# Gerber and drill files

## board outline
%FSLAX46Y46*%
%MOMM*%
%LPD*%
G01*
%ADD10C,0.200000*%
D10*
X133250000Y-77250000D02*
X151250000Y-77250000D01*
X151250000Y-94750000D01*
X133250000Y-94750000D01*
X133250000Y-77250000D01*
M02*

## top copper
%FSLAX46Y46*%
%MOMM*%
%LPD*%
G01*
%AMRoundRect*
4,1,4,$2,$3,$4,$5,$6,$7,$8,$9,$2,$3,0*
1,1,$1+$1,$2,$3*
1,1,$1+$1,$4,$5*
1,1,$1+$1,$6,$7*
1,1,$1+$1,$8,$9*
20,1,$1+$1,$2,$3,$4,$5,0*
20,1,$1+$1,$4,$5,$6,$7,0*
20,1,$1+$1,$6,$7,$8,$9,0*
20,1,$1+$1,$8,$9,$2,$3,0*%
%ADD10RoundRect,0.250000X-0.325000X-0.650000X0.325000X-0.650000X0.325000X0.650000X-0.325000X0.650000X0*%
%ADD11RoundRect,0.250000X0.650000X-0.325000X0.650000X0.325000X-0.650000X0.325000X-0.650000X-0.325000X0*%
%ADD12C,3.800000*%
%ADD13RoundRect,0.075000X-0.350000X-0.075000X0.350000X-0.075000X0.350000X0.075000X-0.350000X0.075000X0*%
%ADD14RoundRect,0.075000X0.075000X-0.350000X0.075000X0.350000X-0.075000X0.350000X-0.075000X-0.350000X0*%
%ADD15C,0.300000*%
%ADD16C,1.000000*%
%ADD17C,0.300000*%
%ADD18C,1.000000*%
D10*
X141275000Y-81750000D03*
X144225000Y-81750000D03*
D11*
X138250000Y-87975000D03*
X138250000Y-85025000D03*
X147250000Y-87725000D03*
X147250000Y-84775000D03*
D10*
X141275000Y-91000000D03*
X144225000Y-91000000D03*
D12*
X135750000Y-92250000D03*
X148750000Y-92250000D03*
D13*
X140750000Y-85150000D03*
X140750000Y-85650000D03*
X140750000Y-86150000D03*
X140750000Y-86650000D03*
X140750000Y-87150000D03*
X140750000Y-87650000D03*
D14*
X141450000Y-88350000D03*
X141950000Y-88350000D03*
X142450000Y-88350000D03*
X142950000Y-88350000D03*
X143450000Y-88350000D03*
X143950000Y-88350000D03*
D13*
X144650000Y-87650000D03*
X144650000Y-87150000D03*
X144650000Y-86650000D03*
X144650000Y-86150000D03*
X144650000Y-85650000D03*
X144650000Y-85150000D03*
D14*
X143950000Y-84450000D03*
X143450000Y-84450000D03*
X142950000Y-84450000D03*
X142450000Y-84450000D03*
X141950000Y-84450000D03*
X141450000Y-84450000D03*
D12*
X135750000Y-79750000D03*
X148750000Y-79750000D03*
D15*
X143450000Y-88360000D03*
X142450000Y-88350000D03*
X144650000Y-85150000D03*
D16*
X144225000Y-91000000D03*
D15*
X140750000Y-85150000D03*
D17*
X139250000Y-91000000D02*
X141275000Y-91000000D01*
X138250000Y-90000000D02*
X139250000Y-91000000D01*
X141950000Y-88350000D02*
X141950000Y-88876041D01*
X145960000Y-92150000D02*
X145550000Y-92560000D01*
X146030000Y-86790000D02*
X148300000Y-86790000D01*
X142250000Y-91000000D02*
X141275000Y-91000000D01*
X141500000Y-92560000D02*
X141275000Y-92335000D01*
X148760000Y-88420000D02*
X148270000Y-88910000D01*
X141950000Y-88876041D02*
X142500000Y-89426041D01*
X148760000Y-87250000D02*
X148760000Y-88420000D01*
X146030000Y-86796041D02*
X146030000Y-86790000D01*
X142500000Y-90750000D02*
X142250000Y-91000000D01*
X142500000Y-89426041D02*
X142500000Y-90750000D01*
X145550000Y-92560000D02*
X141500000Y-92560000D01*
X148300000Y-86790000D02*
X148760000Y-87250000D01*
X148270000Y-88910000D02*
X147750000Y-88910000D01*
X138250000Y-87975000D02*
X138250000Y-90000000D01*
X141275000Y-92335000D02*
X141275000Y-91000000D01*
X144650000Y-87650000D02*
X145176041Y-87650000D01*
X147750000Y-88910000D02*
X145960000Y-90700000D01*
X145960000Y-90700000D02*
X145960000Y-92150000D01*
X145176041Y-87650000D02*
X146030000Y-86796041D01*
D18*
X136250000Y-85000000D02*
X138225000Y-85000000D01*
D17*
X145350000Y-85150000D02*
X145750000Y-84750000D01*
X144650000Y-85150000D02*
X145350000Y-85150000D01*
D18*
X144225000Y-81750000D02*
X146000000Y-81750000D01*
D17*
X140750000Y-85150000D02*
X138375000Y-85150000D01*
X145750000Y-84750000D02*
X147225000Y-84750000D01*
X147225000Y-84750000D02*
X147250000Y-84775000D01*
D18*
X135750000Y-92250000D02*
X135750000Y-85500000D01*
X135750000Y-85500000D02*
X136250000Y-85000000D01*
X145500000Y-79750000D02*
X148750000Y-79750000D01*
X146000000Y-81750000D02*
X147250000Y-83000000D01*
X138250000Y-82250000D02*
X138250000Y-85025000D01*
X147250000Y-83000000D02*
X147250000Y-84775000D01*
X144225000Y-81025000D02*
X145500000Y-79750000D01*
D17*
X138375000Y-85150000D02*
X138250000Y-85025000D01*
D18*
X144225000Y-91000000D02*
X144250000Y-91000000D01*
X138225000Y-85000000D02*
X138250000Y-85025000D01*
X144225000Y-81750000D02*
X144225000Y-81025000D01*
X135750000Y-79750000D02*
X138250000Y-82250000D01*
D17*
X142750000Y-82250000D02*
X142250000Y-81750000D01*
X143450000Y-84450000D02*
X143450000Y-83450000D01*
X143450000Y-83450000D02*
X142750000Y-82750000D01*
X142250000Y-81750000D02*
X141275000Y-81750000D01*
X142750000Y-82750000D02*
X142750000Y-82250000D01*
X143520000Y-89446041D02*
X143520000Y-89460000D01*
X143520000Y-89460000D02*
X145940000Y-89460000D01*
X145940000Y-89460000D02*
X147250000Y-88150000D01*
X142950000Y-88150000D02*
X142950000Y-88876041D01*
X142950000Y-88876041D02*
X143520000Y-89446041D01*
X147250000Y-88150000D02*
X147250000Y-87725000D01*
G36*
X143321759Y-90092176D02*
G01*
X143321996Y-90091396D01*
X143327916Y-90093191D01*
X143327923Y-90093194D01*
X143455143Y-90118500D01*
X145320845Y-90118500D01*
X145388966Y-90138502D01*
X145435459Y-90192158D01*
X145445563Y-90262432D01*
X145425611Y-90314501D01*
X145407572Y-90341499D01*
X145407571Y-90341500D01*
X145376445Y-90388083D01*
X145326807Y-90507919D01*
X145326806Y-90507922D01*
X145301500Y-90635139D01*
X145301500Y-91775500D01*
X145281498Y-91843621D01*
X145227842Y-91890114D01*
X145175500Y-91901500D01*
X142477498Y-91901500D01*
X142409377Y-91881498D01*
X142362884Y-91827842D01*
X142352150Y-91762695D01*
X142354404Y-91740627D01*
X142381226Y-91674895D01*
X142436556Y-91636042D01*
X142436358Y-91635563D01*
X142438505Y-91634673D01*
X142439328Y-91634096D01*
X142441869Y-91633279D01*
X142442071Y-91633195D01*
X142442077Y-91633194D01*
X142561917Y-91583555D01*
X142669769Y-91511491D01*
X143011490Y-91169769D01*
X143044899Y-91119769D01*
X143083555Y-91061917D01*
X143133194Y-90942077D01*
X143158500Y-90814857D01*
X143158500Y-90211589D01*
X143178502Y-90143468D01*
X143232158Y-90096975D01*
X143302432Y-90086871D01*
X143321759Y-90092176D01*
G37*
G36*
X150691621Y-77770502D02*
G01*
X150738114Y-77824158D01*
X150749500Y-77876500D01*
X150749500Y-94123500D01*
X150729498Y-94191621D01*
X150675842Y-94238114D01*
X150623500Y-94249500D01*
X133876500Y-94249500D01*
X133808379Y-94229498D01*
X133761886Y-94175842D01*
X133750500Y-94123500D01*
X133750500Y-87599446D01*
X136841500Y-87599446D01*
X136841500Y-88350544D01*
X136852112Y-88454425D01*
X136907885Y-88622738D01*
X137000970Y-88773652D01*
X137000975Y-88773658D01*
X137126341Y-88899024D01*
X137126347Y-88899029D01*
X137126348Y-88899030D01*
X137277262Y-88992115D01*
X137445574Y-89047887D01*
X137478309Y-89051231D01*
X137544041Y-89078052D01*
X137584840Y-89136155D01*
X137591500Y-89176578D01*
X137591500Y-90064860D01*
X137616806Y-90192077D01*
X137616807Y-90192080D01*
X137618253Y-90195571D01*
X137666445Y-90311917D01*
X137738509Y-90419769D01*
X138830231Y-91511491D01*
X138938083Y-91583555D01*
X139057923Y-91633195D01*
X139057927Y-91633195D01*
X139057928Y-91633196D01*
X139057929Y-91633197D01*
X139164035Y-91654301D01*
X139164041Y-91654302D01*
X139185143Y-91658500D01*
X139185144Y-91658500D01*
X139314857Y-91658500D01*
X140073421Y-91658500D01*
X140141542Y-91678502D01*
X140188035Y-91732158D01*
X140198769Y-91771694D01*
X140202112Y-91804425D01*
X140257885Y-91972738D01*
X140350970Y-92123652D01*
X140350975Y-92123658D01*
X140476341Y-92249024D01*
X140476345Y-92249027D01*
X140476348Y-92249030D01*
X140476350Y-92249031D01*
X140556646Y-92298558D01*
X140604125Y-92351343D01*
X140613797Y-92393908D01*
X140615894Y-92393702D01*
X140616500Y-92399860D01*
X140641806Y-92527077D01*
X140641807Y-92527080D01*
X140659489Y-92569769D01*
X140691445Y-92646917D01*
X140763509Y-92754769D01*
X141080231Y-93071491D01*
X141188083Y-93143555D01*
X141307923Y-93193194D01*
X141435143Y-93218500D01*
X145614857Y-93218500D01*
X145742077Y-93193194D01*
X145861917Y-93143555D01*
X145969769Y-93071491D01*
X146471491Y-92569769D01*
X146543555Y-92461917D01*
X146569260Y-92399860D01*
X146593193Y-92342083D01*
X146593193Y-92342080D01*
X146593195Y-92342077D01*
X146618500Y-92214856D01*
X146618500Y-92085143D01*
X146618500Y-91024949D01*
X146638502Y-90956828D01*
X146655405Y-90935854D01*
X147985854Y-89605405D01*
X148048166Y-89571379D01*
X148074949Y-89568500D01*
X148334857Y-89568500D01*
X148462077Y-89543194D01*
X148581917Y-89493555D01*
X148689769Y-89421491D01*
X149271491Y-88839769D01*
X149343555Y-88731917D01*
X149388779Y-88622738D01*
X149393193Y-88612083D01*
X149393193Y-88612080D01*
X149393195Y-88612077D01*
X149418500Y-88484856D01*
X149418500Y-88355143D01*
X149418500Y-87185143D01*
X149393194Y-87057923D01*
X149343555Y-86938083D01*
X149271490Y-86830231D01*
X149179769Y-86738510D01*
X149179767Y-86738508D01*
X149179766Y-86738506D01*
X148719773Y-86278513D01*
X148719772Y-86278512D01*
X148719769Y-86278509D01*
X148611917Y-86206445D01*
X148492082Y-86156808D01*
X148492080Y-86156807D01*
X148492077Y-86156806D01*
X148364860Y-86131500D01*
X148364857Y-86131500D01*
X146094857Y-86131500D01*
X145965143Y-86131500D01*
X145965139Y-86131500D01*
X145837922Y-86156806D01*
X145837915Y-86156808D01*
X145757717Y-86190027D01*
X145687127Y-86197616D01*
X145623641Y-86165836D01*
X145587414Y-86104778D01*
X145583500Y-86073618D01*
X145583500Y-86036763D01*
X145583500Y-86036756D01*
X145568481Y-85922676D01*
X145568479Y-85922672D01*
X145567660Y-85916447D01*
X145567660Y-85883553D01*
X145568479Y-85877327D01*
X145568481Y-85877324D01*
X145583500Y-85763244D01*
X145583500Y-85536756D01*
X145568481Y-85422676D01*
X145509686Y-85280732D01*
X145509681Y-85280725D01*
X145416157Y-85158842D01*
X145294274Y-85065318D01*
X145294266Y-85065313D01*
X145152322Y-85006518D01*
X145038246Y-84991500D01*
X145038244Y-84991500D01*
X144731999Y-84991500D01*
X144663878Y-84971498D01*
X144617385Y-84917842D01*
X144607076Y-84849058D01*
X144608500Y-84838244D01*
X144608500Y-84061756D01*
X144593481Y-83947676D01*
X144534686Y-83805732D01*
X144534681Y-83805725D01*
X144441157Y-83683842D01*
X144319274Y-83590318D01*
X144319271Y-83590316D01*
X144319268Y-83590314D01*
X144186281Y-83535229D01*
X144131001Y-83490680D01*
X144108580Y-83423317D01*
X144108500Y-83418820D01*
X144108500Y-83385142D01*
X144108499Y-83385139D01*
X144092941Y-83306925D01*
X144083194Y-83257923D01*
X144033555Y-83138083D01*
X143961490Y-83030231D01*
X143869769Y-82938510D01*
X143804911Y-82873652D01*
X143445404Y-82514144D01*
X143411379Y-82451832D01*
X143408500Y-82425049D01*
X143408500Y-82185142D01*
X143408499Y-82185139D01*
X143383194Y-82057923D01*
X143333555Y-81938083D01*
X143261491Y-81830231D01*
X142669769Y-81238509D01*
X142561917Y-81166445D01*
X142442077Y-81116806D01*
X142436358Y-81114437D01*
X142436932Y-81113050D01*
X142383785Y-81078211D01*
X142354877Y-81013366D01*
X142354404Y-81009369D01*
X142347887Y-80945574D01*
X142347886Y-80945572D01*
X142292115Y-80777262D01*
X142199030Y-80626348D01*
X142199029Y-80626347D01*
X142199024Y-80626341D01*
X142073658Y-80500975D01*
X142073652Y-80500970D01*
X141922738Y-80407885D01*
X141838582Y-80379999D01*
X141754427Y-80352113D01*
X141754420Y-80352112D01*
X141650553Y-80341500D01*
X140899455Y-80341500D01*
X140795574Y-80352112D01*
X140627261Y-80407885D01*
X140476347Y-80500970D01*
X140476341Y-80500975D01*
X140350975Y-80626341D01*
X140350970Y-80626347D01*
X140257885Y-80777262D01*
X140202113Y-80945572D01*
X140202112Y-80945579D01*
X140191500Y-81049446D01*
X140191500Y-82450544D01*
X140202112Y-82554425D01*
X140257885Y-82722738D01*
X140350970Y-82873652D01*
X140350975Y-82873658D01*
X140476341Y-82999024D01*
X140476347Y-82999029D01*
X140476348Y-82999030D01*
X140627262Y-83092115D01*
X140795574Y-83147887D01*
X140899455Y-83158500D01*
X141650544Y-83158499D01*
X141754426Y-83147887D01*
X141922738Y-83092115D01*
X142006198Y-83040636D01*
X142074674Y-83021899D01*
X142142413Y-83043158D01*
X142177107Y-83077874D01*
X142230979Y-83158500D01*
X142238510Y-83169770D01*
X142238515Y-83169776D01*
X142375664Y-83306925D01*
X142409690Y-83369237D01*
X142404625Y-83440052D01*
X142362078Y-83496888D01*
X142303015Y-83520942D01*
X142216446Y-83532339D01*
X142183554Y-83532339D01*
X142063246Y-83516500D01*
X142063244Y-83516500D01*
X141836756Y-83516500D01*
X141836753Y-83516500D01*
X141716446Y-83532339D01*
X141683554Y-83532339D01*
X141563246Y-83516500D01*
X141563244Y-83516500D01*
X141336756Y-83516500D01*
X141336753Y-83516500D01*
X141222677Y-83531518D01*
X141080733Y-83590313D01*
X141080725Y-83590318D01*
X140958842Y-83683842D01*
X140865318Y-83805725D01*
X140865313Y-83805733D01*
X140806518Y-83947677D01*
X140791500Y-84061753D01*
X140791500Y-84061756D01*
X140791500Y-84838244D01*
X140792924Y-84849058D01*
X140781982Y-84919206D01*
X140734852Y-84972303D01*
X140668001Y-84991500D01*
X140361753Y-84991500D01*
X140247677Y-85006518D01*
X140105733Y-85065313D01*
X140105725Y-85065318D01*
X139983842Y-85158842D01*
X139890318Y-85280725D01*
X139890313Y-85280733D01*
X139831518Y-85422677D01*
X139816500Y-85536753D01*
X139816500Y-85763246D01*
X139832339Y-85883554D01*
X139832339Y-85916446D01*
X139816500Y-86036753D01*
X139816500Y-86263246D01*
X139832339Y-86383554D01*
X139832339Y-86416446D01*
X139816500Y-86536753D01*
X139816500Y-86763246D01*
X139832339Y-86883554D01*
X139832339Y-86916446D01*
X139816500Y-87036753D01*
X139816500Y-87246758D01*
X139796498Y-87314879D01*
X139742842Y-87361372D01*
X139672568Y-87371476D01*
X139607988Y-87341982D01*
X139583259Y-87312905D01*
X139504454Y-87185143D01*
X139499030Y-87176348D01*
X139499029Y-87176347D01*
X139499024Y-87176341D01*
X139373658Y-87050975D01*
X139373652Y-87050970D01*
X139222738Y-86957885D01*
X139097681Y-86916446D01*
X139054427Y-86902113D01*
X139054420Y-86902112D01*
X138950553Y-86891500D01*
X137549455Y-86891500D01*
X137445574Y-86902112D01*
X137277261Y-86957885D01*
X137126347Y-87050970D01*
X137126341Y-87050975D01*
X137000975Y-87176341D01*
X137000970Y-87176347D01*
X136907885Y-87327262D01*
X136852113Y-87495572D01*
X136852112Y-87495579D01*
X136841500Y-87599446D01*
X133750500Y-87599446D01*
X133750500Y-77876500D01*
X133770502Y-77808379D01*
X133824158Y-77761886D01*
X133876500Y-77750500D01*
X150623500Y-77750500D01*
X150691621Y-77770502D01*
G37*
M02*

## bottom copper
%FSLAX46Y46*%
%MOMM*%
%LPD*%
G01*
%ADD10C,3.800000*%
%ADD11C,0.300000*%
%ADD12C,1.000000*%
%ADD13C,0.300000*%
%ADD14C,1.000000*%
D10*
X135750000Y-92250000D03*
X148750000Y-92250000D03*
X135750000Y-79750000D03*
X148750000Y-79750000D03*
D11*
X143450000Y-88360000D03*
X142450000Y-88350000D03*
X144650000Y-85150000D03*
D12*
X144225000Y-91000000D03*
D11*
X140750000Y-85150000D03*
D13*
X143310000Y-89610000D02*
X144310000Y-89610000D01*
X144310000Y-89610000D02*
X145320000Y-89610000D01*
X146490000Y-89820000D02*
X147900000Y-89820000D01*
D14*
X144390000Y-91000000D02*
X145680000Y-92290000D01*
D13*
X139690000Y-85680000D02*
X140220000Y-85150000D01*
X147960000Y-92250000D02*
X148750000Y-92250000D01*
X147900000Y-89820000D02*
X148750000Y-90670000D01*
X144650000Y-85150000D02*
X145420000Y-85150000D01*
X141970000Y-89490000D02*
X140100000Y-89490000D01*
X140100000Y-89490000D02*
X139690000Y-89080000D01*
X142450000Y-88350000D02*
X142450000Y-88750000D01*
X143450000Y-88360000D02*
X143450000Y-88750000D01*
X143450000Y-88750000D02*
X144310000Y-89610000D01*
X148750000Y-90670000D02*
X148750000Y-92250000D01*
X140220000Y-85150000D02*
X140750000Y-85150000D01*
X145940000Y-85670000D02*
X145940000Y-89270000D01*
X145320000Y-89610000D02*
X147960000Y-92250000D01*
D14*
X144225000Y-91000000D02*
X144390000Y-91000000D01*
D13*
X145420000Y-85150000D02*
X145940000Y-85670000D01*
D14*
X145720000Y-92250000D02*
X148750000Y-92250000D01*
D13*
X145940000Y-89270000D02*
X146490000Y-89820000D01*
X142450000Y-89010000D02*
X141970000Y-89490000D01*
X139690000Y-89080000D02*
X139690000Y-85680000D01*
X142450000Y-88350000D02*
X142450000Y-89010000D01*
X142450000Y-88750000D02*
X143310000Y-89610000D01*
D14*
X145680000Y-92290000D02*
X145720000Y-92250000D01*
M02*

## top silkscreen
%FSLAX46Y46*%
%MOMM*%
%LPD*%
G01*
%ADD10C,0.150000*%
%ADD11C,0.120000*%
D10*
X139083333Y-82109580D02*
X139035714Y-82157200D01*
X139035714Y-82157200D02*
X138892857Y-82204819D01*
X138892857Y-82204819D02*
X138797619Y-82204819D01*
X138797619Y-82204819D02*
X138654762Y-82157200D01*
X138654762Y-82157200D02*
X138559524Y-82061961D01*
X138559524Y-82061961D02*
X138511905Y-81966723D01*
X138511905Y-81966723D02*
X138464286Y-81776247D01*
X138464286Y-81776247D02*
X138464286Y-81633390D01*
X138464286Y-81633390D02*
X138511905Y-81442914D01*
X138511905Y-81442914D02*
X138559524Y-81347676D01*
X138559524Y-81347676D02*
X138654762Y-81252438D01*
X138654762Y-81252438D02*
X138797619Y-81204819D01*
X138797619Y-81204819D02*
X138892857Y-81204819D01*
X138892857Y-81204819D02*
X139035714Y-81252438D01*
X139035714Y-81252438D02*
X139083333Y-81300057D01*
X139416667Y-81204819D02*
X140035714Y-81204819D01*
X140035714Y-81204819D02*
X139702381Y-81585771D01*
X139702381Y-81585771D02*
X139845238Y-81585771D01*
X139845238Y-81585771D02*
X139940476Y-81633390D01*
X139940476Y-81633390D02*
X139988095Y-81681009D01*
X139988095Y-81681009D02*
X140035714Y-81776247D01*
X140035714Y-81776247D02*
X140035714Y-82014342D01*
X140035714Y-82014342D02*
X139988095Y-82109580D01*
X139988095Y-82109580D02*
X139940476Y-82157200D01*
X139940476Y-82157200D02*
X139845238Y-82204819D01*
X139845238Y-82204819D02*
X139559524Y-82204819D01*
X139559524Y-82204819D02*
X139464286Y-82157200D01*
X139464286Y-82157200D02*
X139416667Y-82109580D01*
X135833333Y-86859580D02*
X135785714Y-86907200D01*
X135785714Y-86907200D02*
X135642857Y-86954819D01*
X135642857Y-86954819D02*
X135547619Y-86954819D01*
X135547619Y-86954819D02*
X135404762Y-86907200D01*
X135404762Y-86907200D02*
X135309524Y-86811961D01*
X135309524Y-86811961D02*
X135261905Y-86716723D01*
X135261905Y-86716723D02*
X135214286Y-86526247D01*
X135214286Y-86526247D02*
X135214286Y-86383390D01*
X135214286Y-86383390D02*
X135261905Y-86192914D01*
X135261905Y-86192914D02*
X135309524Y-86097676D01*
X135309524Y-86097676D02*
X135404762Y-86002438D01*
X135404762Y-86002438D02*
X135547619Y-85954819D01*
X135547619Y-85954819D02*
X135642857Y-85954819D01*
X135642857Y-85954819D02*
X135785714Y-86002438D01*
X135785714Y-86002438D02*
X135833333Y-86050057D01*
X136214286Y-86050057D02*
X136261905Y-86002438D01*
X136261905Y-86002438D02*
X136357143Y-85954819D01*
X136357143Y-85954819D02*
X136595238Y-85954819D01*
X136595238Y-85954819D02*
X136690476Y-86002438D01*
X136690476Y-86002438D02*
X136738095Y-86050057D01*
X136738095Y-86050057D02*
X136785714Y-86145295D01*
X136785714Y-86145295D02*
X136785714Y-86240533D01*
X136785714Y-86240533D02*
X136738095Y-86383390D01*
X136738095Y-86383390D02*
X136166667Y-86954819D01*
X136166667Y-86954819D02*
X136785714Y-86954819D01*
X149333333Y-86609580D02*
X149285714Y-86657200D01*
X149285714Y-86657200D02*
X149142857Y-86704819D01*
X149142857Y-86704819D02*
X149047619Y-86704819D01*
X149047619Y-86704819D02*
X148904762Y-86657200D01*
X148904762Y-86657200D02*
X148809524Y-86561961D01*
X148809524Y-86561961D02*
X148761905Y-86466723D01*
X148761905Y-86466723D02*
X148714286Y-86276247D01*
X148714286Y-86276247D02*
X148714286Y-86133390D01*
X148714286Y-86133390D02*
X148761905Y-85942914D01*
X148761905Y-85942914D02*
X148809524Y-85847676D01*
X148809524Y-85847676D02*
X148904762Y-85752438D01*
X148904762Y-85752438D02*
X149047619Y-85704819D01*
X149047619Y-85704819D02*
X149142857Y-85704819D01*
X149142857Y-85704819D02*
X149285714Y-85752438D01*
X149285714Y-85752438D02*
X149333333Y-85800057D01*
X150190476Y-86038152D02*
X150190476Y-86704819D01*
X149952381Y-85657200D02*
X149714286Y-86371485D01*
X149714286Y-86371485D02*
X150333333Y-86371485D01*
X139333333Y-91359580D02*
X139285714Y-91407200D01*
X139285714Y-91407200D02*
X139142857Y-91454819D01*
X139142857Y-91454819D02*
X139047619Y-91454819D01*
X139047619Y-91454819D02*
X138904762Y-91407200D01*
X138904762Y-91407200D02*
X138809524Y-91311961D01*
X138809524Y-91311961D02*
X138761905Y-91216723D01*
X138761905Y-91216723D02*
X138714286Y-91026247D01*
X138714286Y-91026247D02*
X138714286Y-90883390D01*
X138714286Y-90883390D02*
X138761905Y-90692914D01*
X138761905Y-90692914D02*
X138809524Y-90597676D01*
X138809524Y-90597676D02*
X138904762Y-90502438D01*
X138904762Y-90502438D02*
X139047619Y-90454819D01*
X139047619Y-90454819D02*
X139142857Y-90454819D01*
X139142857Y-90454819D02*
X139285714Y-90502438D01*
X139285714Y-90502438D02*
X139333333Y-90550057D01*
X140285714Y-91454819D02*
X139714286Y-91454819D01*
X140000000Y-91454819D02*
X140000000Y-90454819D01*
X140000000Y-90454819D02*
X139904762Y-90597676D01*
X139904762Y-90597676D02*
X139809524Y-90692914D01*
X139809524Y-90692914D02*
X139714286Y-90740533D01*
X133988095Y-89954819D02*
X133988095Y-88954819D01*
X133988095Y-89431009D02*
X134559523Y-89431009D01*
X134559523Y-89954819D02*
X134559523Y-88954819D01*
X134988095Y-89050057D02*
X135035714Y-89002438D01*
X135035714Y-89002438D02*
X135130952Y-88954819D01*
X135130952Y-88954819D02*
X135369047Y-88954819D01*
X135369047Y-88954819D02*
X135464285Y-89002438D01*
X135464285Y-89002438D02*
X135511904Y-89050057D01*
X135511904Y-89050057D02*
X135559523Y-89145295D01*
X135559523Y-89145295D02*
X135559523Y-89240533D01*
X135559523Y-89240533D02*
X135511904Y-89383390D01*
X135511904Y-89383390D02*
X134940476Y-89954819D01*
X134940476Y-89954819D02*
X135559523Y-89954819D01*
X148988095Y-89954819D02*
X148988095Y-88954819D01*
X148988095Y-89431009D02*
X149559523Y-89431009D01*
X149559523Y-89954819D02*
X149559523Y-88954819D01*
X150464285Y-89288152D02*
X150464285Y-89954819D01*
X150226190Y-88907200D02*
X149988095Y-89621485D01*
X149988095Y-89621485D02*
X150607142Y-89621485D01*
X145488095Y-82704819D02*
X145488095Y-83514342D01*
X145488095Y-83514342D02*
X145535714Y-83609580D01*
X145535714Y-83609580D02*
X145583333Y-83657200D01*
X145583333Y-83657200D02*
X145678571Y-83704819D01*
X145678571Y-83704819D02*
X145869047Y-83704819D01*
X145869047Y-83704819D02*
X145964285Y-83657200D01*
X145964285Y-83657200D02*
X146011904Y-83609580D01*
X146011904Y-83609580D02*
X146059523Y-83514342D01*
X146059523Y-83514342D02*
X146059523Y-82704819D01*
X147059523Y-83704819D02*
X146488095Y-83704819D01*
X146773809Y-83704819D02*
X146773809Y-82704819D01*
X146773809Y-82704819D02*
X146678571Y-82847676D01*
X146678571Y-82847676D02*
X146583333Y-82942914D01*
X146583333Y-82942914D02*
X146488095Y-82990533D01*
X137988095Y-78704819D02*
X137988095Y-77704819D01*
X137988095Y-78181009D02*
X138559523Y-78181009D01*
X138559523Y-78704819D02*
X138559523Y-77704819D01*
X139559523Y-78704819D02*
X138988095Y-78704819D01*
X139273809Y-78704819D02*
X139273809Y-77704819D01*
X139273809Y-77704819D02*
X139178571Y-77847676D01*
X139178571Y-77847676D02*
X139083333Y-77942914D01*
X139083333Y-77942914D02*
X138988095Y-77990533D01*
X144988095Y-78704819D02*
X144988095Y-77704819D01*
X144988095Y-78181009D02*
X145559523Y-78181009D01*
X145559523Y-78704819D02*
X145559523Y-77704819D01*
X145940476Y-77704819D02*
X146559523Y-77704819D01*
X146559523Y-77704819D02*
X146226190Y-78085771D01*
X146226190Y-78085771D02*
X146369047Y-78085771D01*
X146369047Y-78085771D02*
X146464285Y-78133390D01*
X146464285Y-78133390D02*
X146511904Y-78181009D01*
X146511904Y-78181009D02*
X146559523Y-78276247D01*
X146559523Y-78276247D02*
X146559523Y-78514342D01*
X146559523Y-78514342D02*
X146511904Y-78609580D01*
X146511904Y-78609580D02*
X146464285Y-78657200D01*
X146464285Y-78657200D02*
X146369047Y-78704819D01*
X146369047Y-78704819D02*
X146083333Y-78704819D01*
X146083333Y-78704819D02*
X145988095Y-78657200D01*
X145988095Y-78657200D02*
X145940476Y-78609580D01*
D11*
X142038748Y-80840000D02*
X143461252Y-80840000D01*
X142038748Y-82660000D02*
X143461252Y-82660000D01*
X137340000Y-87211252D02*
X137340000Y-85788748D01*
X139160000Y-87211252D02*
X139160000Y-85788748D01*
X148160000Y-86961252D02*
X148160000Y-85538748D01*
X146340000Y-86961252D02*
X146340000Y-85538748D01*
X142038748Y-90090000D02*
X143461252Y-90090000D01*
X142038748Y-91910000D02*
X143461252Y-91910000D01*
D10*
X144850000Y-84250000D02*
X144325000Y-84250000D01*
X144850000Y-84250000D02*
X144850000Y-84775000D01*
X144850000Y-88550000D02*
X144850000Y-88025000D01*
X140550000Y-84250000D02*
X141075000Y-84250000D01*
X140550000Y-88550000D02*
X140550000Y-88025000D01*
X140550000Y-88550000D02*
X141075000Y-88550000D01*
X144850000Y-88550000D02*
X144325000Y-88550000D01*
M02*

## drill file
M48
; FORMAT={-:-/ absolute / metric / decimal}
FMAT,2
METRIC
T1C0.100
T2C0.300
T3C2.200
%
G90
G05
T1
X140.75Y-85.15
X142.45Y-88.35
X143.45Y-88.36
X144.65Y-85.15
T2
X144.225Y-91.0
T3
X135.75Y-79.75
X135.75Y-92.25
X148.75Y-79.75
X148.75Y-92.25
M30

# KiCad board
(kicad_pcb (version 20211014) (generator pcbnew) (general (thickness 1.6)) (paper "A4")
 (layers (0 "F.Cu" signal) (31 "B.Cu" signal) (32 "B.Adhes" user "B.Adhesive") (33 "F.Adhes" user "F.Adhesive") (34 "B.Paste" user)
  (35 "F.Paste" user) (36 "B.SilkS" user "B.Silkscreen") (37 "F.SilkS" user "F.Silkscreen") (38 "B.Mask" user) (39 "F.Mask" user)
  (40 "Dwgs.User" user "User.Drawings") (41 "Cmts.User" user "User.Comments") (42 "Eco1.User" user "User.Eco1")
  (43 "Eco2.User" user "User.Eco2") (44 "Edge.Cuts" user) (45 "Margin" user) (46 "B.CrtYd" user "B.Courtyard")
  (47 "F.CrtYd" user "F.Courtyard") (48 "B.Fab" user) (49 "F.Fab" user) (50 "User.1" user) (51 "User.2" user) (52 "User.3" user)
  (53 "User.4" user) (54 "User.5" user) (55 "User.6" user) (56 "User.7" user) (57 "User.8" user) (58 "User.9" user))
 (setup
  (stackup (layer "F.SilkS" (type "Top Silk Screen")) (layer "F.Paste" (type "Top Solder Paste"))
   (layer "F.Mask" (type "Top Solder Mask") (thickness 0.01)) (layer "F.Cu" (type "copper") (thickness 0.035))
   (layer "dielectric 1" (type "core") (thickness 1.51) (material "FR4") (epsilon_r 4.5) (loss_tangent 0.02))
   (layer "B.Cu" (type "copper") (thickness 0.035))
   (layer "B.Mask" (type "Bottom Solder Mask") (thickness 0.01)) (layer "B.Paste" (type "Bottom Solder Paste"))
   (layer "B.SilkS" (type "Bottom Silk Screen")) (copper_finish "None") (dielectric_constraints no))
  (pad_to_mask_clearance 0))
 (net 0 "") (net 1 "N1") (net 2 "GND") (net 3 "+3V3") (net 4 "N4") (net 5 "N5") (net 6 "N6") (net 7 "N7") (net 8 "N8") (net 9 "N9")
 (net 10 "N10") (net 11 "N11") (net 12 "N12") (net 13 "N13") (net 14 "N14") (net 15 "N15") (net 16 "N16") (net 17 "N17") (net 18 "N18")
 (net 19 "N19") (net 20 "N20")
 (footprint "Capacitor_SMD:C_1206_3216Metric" (layer "F.Cu") (at 142.75 81.75)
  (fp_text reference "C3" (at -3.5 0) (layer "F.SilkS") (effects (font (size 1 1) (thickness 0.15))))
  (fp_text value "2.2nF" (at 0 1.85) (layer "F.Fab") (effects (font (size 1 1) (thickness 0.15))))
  (fp_line (start -0.711252 -0.91) (end 0.711252 -0.91) (layer "F.SilkS") (width 0.12))
  (fp_line (start -0.711252 0.91) (end 0.711252 0.91) (layer "F.SilkS") (width 0.12))
  (pad "1" smd roundrect (at -1.475 0) (size 1.15 1.8) (layers "F.Cu" "F.Paste" "F.Mask") (roundrect_rratio 0.217391) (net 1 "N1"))
  (pad "2" smd roundrect (at 1.475 0) (size 1.15 1.8) (layers "F.Cu" "F.Paste" "F.Mask") (roundrect_rratio 0.217391) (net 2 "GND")))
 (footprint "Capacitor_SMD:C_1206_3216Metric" (layer "F.Cu") (at 138.25 86.5 90)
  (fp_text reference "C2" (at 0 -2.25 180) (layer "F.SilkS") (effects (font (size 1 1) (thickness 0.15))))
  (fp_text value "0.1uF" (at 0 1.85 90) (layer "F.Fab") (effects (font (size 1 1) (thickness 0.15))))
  (fp_line (start -0.711252 -0.91) (end 0.711252 -0.91) (layer "F.SilkS") (width 0.12))
  (fp_line (start -0.711252 0.91) (end 0.711252 0.91) (layer "F.SilkS") (width 0.12))
  (pad "1" smd roundrect (at -1.475 0 90) (size 1.15 1.8) (layers "F.Cu" "F.Paste" "F.Mask") (roundrect_rratio 0.217391) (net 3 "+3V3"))
  (pad "2" smd roundrect (at 1.475 0 90) (size 1.15 1.8) (layers "F.Cu" "F.Paste" "F.Mask") (roundrect_rratio 0.217391) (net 2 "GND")))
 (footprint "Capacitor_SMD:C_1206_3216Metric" (layer "F.Cu") (at 147.25 86.25 90)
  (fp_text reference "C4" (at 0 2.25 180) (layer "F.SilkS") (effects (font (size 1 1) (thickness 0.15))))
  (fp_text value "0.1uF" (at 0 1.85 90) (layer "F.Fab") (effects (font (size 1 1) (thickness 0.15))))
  (fp_line (start -0.711252 0.91) (end 0.711252 0.91) (layer "F.SilkS") (width 0.12))
  (fp_line (start -0.711252 -0.91) (end 0.711252 -0.91) (layer "F.SilkS") (width 0.12))
  (pad "1" smd roundrect (at -1.475 0 90) (size 1.15 1.8) (layers "F.Cu" "F.Paste" "F.Mask") (roundrect_rratio 0.217391) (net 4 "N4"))
  (pad "2" smd roundrect (at 1.475 0 90) (size 1.15 1.8) (layers "F.Cu" "F.Paste" "F.Mask") (roundrect_rratio 0.217391) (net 2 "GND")))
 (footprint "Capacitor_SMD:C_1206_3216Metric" (layer "F.Cu") (at 142.75 91)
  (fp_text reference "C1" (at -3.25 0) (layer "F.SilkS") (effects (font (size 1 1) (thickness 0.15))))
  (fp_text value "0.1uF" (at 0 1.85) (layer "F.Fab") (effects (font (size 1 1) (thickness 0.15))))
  (fp_line (start -0.711252 -0.91) (end 0.711252 -0.91) (layer "F.SilkS") (width 0.12))
  (fp_line (start -0.711252 0.91) (end 0.711252 0.91) (layer "F.SilkS") (width 0.12))
  (pad "1" smd roundrect (at -1.475 0) (size 1.15 1.8) (layers "F.Cu" "F.Paste" "F.Mask") (roundrect_rratio 0.217391) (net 3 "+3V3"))
  (pad "2" smd roundrect (at 1.475 0) (size 1.15 1.8) (layers "F.Cu" "F.Paste" "F.Mask") (roundrect_rratio 0.217391) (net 2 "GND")))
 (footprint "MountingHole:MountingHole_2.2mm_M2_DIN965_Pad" (layer "F.Cu") (at 135.75 92.25)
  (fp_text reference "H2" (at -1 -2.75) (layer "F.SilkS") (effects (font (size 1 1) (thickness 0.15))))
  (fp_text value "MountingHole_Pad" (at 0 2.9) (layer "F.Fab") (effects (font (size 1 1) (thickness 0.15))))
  (pad "1" thru_hole circle (at 0 0) (size 3.8 3.8) (drill 2.2) (layers *.Cu *.Mask) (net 2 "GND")))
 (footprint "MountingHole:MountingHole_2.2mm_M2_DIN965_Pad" (layer "F.Cu") (at 148.75 92.25)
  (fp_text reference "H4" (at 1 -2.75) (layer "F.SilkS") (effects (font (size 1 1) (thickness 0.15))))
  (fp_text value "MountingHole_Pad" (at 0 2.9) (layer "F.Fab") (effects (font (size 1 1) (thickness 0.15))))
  (pad "1" thru_hole circle (at 0 0) (size 3.8 3.8) (drill 2.2) (layers *.Cu *.Mask) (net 2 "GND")))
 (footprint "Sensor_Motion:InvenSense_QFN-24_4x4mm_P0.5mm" (layer "F.Cu") (at 142.7 86.4)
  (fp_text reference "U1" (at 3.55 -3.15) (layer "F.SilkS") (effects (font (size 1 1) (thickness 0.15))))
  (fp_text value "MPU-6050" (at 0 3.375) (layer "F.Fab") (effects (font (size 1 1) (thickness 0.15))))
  (fp_line (start 2.15 -2.15) (end 1.625 -2.15) (layer "F.SilkS") (width 0.15))
  (fp_line (start 2.15 -2.15) (end 2.15 -1.625) (layer "F.SilkS") (width 0.15))
  (fp_line (start 2.15 2.15) (end 2.15 1.625) (layer "F.SilkS") (width 0.15))
  (fp_line (start -2.15 -2.15) (end -1.625 -2.15) (layer "F.SilkS") (width 0.15))
  (fp_line (start -2.15 2.15) (end -2.15 1.625) (layer "F.SilkS") (width 0.15))
  (fp_line (start -2.15 2.15) (end -1.625 2.15) (layer "F.SilkS") (width 0.15))
  (fp_line (start 2.15 2.15) (end 1.625 2.15) (layer "F.SilkS") (width 0.15))
  (pad "1" smd roundrect (at -1.95 -1.25) (size 0.85 0.3) (layers "F.Cu" "F.Paste" "F.Mask") (roundrect_rratio 0.25) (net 2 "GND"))
  (pad "2" smd roundrect (at -1.95 -0.75) (size 0.85 0.3) (layers "F.Cu" "F.Paste" "F.Mask") (roundrect_rratio 0.25) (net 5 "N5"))
  (pad "3" smd roundrect (at -1.95 -0.25) (size 0.85 0.3) (layers "F.Cu" "F.Paste" "F.Mask") (roundrect_rratio 0.25) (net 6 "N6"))
  (pad "4" smd roundrect (at -1.95 0.25) (size 0.85 0.3) (layers "F.Cu" "F.Paste" "F.Mask") (roundrect_rratio 0.25) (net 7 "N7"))
  (pad "5" smd roundrect (at -1.95 0.75) (size 0.85 0.3) (layers "F.Cu" "F.Paste" "F.Mask") (roundrect_rratio 0.25) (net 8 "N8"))
  (pad "6" smd roundrect (at -1.95 1.25) (size 0.85 0.3) (layers "F.Cu" "F.Paste" "F.Mask") (roundrect_rratio 0.25) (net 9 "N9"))
  (pad "7" smd roundrect (at -1.25 1.95 90) (size 0.85 0.3) (layers "F.Cu" "F.Paste" "F.Mask") (roundrect_rratio 0.25) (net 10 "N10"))
  (pad "8" smd roundrect (at -0.75 1.95 90) (size 0.85 0.3) (layers "F.Cu" "F.Paste" "F.Mask") (roundrect_rratio 0.25) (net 3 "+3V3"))
  (pad "9" smd roundrect (at -0.25 1.95 90) (size 0.85 0.3) (layers "F.Cu" "F.Paste" "F.Mask") (roundrect_rratio 0.25) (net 2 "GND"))
  (pad "10" smd roundrect (at 0.25 1.95 90) (size 0.85 0.3) (layers "F.Cu" "F.Paste" "F.Mask") (roundrect_rratio 0.25) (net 4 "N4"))
  (pad "11" smd roundrect (at 0.75 1.95 90) (size 0.85 0.3) (layers "F.Cu" "F.Paste" "F.Mask") (roundrect_rratio 0.25) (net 2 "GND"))
  (pad "12" smd roundrect (at 1.25 1.95 90) (size 0.85 0.3) (layers "F.Cu" "F.Paste" "F.Mask") (roundrect_rratio 0.25) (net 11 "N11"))
  (pad "13" smd roundrect (at 1.95 1.25) (size 0.85 0.3) (layers "F.Cu" "F.Paste" "F.Mask") (roundrect_rratio 0.25) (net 3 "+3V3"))
  (pad "14" smd roundrect (at 1.95 0.75) (size 0.85 0.3) (layers "F.Cu" "F.Paste" "F.Mask") (roundrect_rratio 0.25) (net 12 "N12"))
  (pad "15" smd roundrect (at 1.95 0.25) (size 0.85 0.3) (layers "F.Cu" "F.Paste" "F.Mask") (roundrect_rratio 0.25) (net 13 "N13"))
  (pad "16" smd roundrect (at 1.95 -0.25) (size 0.85 0.3) (layers "F.Cu" "F.Paste" "F.Mask") (roundrect_rratio 0.25) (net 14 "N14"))
  (pad "17" smd roundrect (at 1.95 -0.75) (size 0.85 0.3) (layers "F.Cu" "F.Paste" "F.Mask") (roundrect_rratio 0.25) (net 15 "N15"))
  (pad "18" smd roundrect (at 1.95 -1.25) (size 0.85 0.3) (layers "F.Cu" "F.Paste" "F.Mask") (roundrect_rratio 0.25) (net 2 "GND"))
  (pad "19" smd roundrect (at 1.25 -1.95 90) (size 0.85 0.3) (layers "F.Cu" "F.Paste" "F.Mask") (roundrect_rratio 0.25) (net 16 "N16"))
  (pad "20" smd roundrect (at 0.75 -1.95 90) (size 0.85 0.3) (layers "F.Cu" "F.Paste" "F.Mask") (roundrect_rratio 0.25) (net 1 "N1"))
  (pad "21" smd roundrect (at 0.25 -1.95 90) (size 0.85 0.3) (layers "F.Cu" "F.Paste" "F.Mask") (roundrect_rratio 0.25) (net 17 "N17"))
  (pad "22" smd roundrect (at -0.25 -1.95 90) (size 0.85 0.3) (layers "F.Cu" "F.Paste" "F.Mask") (roundrect_rratio 0.25) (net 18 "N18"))
  (pad "23" smd roundrect (at -0.75 -1.95 90) (size 0.85 0.3) (layers "F.Cu" "F.Paste" "F.Mask") (roundrect_rratio 0.25) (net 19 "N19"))
  (pad "24" smd roundrect (at -1.25 -1.95 90) (size 0.85 0.3) (layers "F.Cu" "F.Paste" "F.Mask") (roundrect_rratio 0.25) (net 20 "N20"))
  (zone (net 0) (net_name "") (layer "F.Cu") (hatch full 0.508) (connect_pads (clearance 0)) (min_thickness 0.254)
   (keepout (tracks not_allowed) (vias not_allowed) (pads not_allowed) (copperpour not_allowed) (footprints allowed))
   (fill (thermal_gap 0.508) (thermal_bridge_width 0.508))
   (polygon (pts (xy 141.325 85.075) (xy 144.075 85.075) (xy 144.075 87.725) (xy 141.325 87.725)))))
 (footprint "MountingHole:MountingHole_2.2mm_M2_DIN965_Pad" (layer "F.Cu") (at 135.75 79.75)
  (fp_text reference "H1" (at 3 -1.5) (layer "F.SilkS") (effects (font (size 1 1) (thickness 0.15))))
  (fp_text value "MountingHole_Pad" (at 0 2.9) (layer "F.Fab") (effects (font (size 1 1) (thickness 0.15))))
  (pad "1" thru_hole circle (at 0 0) (size 3.8 3.8) (drill 2.2) (layers *.Cu *.Mask) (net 2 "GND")))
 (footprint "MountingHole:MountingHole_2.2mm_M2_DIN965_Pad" (layer "F.Cu") (at 148.75 79.75)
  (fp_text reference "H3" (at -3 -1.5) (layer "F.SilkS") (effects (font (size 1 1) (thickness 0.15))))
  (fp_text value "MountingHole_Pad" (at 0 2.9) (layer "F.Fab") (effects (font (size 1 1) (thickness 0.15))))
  (pad "1" thru_hole circle (at 0 0) (size 3.8 3.8) (drill 2.2) (layers *.Cu *.Mask) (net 2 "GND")))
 (gr_rect (start 133.25 77.25) (end 151.25 94.75) (layer "Edge.Cuts") (width 0.2) (fill none))
 (segment (start 139.25 91) (end 141.275 91) (width 0.3) (layer "F.Cu") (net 3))
 (segment (start 138.25 90) (end 139.25 91) (width 0.3) (layer "F.Cu") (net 3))
 (segment (start 141.95 88.35) (end 141.95 88.876041) (width 0.3) (layer "F.Cu") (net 3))
 (segment (start 145.96 92.15) (end 145.55 92.56) (width 0.3) (layer "F.Cu") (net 3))
 (segment (start 146.03 86.79) (end 148.3 86.79) (width 0.3) (layer "F.Cu") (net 3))
 (segment (start 142.25 91) (end 141.275 91) (width 0.3) (layer "F.Cu") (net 3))
 (segment (start 141.5 92.56) (end 141.275 92.335) (width 0.3) (layer "F.Cu") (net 3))
 (segment (start 148.76 88.42) (end 148.27 88.91) (width 0.3) (layer "F.Cu") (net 3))
 (segment (start 141.95 88.876041) (end 142.5 89.426041) (width 0.3) (layer "F.Cu") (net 3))
 (segment (start 148.76 87.25) (end 148.76 88.42) (width 0.3) (layer "F.Cu") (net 3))
 (segment (start 146.03 86.796041) (end 146.03 86.79) (width 0.3) (layer "F.Cu") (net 3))
 (segment (start 142.5 90.75) (end 142.25 91) (width 0.3) (layer "F.Cu") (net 3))
 (segment (start 142.5 89.426041) (end 142.5 90.75) (width 0.3) (layer "F.Cu") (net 3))
 (segment (start 145.55 92.56) (end 141.5 92.56) (width 0.3) (layer "F.Cu") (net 3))
 (segment (start 148.3 86.79) (end 148.76 87.25) (width 0.3) (layer "F.Cu") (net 3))
 (segment (start 148.27 88.91) (end 147.75 88.91) (width 0.3) (layer "F.Cu") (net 3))
 (segment (start 138.25 87.975) (end 138.25 90) (width 0.3) (layer "F.Cu") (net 3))
 (segment (start 141.275 92.335) (end 141.275 91) (width 0.3) (layer "F.Cu") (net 3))
 (segment (start 144.65 87.65) (end 145.176041 87.65) (width 0.3) (layer "F.Cu") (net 3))
 (segment (start 147.75 88.91) (end 145.96 90.7) (width 0.3) (layer "F.Cu") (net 3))
 (segment (start 145.96 90.7) (end 145.96 92.15) (width 0.3) (layer "F.Cu") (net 3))
 (segment (start 145.176041 87.65) (end 146.03 86.796041) (width 0.3) (layer "F.Cu") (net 3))
 (segment (start 136.25 85) (end 138.225 85) (width 1) (layer "F.Cu") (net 2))
 (segment (start 145.35 85.15) (end 145.75 84.75) (width 0.3) (layer "F.Cu") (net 2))
 (segment (start 144.65 85.15) (end 145.35 85.15) (width 0.3) (layer "F.Cu") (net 2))
 (segment (start 144.225 81.75) (end 146 81.75) (width 1) (layer "F.Cu") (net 2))
 (segment (start 140.75 85.15) (end 138.375 85.15) (width 0.3) (layer "F.Cu") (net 2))
 (segment (start 145.75 84.75) (end 147.225 84.75) (width 0.3) (layer "F.Cu") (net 2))
 (segment (start 147.225 84.75) (end 147.25 84.775) (width 0.3) (layer "F.Cu") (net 2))
 (segment (start 135.75 92.25) (end 135.75 85.5) (width 1) (layer "F.Cu") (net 2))
 (segment (start 135.75 85.5) (end 136.25 85) (width 1) (layer "F.Cu") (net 2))
 (segment (start 145.5 79.75) (end 148.75 79.75) (width 1) (layer "F.Cu") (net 2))
 (segment (start 146 81.75) (end 147.25 83) (width 1) (layer "F.Cu") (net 2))
 (segment (start 138.25 82.25) (end 138.25 85.025) (width 1) (layer "F.Cu") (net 2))
 (segment (start 147.25 83) (end 147.25 84.775) (width 1) (layer "F.Cu") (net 2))
 (segment (start 144.225 81.025) (end 145.5 79.75) (width 1) (layer "F.Cu") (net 2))
 (segment (start 138.375 85.15) (end 138.25 85.025) (width 0.3) (layer "F.Cu") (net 2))
 (segment (start 144.225 91) (end 144.25 91) (width 1) (layer "F.Cu") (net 2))
 (segment (start 138.225 85) (end 138.25 85.025) (width 1) (layer "F.Cu") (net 2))
 (segment (start 144.225 81.75) (end 144.225 81.025) (width 1) (layer "F.Cu") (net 2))
 (segment (start 135.75 79.75) (end 138.25 82.25) (width 1) (layer "F.Cu") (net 2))
 (via (at 143.45 88.36) (size 0.3) (drill 0.1) (layers "F.Cu" "B.Cu") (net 2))
 (via (at 142.45 88.35) (size 0.3) (drill 0.1) (layers "F.Cu" "B.Cu") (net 2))
 (via (at 144.65 85.15) (size 0.3) (drill 0.1) (layers "F.Cu" "B.Cu") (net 2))
 (via (at 144.225 91) (size 1) (drill 0.3) (layers "F.Cu" "B.Cu") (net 2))
 (via (at 140.75 85.15) (size 0.3) (drill 0.1) (layers "F.Cu" "B.Cu") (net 2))
 (segment (start 143.31 89.61) (end 144.31 89.61) (width 0.3) (layer "B.Cu") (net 2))
 (segment (start 144.31 89.61) (end 145.32 89.61) (width 0.3) (layer "B.Cu") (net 2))
 (segment (start 146.49 89.82) (end 147.9 89.82) (width 0.3) (layer "B.Cu") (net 2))
 (segment (start 144.39 91) (end 145.68 92.29) (width 1) (layer "B.Cu") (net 2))
 (segment (start 139.69 85.68) (end 140.22 85.15) (width 0.3) (layer "B.Cu") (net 2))
 (segment (start 147.96 92.25) (end 148.75 92.25) (width 0.3) (layer "B.Cu") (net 2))
 (segment (start 147.9 89.82) (end 148.75 90.67) (width 0.3) (layer "B.Cu") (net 2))
 (segment (start 144.65 85.15) (end 145.42 85.15) (width 0.3) (layer "B.Cu") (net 2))
 (segment (start 141.97 89.49) (end 140.1 89.49) (width 0.3) (layer "B.Cu") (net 2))
 (segment (start 140.1 89.49) (end 139.69 89.08) (width 0.3) (layer "B.Cu") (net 2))
 (segment (start 142.45 88.35) (end 142.45 88.75) (width 0.3) (layer "B.Cu") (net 2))
 (segment (start 143.45 88.36) (end 143.45 88.75) (width 0.3) (layer "B.Cu") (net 2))
 (segment (start 143.45 88.75) (end 144.31 89.61) (width 0.3) (layer "B.Cu") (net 2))
 (segment (start 148.75 90.67) (end 148.75 92.25) (width 0.3) (layer "B.Cu") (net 2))
 (segment (start 140.22 85.15) (end 140.75 85.15) (width 0.3) (layer "B.Cu") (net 2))
 (segment (start 145.94 85.67) (end 145.94 89.27) (width 0.3) (layer "B.Cu") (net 2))
 (segment (start 145.32 89.61) (end 147.96 92.25) (width 0.3) (layer "B.Cu") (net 2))
 (segment (start 144.225 91) (end 144.39 91) (width 1) (layer "B.Cu") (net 2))
 (segment (start 145.42 85.15) (end 145.94 85.67) (width 0.3) (layer "B.Cu") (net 2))
 (segment (start 145.72 92.25) (end 148.75 92.25) (width 1) (layer "B.Cu") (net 2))
 (segment (start 145.94 89.27) (end 146.49 89.82) (width 0.3) (layer "B.Cu") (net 2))
 (segment (start 142.45 89.01) (end 141.97 89.49) (width 0.3) (layer "B.Cu") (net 2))
 (segment (start 139.69 89.08) (end 139.69 85.68) (width 0.3) (layer "B.Cu") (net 2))
 (segment (start 142.45 88.35) (end 142.45 89.01) (width 0.3) (layer "B.Cu") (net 2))
 (segment (start 142.45 88.75) (end 143.31 89.61) (width 0.3) (layer "B.Cu") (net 2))
 (segment (start 145.68 92.29) (end 145.72 92.25) (width 1) (layer "B.Cu") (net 2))
 (segment (start 142.75 82.25) (end 142.25 81.75) (width 0.3) (layer "F.Cu") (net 1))
 (segment (start 143.45 84.45) (end 143.45 83.45) (width 0.3) (layer "F.Cu") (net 1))
 (segment (start 143.45 83.45) (end 142.75 82.75) (width 0.3) (layer "F.Cu") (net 1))
 (segment (start 142.25 81.75) (end 141.275 81.75) (width 0.3) (layer "F.Cu") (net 1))
 (segment (start 142.75 82.75) (end 142.75 82.25) (width 0.3) (layer "F.Cu") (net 1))
 (segment (start 143.52 89.446041) (end 143.52 89.46) (width 0.3) (layer "F.Cu") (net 4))
 (segment (start 143.52 89.46) (end 145.94 89.46) (width 0.3) (layer "F.Cu") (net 4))
 (segment (start 145.94 89.46) (end 147.25 88.15) (width 0.3) (layer "F.Cu") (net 4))
 (segment (start 142.95 88.15) (end 142.95 88.876041) (width 0.3) (layer "F.Cu") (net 4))
 (segment (start 142.95 88.876041) (end 143.52 89.446041) (width 0.3) (layer "F.Cu") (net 4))
 (segment (start 147.25 88.15) (end 147.25 87.725) (width 0.3) (layer "F.Cu") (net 4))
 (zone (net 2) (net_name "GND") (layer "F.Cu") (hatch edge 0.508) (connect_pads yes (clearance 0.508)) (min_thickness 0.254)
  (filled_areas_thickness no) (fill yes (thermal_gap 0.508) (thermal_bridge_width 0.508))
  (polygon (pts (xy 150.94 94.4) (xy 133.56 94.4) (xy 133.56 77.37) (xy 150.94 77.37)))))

